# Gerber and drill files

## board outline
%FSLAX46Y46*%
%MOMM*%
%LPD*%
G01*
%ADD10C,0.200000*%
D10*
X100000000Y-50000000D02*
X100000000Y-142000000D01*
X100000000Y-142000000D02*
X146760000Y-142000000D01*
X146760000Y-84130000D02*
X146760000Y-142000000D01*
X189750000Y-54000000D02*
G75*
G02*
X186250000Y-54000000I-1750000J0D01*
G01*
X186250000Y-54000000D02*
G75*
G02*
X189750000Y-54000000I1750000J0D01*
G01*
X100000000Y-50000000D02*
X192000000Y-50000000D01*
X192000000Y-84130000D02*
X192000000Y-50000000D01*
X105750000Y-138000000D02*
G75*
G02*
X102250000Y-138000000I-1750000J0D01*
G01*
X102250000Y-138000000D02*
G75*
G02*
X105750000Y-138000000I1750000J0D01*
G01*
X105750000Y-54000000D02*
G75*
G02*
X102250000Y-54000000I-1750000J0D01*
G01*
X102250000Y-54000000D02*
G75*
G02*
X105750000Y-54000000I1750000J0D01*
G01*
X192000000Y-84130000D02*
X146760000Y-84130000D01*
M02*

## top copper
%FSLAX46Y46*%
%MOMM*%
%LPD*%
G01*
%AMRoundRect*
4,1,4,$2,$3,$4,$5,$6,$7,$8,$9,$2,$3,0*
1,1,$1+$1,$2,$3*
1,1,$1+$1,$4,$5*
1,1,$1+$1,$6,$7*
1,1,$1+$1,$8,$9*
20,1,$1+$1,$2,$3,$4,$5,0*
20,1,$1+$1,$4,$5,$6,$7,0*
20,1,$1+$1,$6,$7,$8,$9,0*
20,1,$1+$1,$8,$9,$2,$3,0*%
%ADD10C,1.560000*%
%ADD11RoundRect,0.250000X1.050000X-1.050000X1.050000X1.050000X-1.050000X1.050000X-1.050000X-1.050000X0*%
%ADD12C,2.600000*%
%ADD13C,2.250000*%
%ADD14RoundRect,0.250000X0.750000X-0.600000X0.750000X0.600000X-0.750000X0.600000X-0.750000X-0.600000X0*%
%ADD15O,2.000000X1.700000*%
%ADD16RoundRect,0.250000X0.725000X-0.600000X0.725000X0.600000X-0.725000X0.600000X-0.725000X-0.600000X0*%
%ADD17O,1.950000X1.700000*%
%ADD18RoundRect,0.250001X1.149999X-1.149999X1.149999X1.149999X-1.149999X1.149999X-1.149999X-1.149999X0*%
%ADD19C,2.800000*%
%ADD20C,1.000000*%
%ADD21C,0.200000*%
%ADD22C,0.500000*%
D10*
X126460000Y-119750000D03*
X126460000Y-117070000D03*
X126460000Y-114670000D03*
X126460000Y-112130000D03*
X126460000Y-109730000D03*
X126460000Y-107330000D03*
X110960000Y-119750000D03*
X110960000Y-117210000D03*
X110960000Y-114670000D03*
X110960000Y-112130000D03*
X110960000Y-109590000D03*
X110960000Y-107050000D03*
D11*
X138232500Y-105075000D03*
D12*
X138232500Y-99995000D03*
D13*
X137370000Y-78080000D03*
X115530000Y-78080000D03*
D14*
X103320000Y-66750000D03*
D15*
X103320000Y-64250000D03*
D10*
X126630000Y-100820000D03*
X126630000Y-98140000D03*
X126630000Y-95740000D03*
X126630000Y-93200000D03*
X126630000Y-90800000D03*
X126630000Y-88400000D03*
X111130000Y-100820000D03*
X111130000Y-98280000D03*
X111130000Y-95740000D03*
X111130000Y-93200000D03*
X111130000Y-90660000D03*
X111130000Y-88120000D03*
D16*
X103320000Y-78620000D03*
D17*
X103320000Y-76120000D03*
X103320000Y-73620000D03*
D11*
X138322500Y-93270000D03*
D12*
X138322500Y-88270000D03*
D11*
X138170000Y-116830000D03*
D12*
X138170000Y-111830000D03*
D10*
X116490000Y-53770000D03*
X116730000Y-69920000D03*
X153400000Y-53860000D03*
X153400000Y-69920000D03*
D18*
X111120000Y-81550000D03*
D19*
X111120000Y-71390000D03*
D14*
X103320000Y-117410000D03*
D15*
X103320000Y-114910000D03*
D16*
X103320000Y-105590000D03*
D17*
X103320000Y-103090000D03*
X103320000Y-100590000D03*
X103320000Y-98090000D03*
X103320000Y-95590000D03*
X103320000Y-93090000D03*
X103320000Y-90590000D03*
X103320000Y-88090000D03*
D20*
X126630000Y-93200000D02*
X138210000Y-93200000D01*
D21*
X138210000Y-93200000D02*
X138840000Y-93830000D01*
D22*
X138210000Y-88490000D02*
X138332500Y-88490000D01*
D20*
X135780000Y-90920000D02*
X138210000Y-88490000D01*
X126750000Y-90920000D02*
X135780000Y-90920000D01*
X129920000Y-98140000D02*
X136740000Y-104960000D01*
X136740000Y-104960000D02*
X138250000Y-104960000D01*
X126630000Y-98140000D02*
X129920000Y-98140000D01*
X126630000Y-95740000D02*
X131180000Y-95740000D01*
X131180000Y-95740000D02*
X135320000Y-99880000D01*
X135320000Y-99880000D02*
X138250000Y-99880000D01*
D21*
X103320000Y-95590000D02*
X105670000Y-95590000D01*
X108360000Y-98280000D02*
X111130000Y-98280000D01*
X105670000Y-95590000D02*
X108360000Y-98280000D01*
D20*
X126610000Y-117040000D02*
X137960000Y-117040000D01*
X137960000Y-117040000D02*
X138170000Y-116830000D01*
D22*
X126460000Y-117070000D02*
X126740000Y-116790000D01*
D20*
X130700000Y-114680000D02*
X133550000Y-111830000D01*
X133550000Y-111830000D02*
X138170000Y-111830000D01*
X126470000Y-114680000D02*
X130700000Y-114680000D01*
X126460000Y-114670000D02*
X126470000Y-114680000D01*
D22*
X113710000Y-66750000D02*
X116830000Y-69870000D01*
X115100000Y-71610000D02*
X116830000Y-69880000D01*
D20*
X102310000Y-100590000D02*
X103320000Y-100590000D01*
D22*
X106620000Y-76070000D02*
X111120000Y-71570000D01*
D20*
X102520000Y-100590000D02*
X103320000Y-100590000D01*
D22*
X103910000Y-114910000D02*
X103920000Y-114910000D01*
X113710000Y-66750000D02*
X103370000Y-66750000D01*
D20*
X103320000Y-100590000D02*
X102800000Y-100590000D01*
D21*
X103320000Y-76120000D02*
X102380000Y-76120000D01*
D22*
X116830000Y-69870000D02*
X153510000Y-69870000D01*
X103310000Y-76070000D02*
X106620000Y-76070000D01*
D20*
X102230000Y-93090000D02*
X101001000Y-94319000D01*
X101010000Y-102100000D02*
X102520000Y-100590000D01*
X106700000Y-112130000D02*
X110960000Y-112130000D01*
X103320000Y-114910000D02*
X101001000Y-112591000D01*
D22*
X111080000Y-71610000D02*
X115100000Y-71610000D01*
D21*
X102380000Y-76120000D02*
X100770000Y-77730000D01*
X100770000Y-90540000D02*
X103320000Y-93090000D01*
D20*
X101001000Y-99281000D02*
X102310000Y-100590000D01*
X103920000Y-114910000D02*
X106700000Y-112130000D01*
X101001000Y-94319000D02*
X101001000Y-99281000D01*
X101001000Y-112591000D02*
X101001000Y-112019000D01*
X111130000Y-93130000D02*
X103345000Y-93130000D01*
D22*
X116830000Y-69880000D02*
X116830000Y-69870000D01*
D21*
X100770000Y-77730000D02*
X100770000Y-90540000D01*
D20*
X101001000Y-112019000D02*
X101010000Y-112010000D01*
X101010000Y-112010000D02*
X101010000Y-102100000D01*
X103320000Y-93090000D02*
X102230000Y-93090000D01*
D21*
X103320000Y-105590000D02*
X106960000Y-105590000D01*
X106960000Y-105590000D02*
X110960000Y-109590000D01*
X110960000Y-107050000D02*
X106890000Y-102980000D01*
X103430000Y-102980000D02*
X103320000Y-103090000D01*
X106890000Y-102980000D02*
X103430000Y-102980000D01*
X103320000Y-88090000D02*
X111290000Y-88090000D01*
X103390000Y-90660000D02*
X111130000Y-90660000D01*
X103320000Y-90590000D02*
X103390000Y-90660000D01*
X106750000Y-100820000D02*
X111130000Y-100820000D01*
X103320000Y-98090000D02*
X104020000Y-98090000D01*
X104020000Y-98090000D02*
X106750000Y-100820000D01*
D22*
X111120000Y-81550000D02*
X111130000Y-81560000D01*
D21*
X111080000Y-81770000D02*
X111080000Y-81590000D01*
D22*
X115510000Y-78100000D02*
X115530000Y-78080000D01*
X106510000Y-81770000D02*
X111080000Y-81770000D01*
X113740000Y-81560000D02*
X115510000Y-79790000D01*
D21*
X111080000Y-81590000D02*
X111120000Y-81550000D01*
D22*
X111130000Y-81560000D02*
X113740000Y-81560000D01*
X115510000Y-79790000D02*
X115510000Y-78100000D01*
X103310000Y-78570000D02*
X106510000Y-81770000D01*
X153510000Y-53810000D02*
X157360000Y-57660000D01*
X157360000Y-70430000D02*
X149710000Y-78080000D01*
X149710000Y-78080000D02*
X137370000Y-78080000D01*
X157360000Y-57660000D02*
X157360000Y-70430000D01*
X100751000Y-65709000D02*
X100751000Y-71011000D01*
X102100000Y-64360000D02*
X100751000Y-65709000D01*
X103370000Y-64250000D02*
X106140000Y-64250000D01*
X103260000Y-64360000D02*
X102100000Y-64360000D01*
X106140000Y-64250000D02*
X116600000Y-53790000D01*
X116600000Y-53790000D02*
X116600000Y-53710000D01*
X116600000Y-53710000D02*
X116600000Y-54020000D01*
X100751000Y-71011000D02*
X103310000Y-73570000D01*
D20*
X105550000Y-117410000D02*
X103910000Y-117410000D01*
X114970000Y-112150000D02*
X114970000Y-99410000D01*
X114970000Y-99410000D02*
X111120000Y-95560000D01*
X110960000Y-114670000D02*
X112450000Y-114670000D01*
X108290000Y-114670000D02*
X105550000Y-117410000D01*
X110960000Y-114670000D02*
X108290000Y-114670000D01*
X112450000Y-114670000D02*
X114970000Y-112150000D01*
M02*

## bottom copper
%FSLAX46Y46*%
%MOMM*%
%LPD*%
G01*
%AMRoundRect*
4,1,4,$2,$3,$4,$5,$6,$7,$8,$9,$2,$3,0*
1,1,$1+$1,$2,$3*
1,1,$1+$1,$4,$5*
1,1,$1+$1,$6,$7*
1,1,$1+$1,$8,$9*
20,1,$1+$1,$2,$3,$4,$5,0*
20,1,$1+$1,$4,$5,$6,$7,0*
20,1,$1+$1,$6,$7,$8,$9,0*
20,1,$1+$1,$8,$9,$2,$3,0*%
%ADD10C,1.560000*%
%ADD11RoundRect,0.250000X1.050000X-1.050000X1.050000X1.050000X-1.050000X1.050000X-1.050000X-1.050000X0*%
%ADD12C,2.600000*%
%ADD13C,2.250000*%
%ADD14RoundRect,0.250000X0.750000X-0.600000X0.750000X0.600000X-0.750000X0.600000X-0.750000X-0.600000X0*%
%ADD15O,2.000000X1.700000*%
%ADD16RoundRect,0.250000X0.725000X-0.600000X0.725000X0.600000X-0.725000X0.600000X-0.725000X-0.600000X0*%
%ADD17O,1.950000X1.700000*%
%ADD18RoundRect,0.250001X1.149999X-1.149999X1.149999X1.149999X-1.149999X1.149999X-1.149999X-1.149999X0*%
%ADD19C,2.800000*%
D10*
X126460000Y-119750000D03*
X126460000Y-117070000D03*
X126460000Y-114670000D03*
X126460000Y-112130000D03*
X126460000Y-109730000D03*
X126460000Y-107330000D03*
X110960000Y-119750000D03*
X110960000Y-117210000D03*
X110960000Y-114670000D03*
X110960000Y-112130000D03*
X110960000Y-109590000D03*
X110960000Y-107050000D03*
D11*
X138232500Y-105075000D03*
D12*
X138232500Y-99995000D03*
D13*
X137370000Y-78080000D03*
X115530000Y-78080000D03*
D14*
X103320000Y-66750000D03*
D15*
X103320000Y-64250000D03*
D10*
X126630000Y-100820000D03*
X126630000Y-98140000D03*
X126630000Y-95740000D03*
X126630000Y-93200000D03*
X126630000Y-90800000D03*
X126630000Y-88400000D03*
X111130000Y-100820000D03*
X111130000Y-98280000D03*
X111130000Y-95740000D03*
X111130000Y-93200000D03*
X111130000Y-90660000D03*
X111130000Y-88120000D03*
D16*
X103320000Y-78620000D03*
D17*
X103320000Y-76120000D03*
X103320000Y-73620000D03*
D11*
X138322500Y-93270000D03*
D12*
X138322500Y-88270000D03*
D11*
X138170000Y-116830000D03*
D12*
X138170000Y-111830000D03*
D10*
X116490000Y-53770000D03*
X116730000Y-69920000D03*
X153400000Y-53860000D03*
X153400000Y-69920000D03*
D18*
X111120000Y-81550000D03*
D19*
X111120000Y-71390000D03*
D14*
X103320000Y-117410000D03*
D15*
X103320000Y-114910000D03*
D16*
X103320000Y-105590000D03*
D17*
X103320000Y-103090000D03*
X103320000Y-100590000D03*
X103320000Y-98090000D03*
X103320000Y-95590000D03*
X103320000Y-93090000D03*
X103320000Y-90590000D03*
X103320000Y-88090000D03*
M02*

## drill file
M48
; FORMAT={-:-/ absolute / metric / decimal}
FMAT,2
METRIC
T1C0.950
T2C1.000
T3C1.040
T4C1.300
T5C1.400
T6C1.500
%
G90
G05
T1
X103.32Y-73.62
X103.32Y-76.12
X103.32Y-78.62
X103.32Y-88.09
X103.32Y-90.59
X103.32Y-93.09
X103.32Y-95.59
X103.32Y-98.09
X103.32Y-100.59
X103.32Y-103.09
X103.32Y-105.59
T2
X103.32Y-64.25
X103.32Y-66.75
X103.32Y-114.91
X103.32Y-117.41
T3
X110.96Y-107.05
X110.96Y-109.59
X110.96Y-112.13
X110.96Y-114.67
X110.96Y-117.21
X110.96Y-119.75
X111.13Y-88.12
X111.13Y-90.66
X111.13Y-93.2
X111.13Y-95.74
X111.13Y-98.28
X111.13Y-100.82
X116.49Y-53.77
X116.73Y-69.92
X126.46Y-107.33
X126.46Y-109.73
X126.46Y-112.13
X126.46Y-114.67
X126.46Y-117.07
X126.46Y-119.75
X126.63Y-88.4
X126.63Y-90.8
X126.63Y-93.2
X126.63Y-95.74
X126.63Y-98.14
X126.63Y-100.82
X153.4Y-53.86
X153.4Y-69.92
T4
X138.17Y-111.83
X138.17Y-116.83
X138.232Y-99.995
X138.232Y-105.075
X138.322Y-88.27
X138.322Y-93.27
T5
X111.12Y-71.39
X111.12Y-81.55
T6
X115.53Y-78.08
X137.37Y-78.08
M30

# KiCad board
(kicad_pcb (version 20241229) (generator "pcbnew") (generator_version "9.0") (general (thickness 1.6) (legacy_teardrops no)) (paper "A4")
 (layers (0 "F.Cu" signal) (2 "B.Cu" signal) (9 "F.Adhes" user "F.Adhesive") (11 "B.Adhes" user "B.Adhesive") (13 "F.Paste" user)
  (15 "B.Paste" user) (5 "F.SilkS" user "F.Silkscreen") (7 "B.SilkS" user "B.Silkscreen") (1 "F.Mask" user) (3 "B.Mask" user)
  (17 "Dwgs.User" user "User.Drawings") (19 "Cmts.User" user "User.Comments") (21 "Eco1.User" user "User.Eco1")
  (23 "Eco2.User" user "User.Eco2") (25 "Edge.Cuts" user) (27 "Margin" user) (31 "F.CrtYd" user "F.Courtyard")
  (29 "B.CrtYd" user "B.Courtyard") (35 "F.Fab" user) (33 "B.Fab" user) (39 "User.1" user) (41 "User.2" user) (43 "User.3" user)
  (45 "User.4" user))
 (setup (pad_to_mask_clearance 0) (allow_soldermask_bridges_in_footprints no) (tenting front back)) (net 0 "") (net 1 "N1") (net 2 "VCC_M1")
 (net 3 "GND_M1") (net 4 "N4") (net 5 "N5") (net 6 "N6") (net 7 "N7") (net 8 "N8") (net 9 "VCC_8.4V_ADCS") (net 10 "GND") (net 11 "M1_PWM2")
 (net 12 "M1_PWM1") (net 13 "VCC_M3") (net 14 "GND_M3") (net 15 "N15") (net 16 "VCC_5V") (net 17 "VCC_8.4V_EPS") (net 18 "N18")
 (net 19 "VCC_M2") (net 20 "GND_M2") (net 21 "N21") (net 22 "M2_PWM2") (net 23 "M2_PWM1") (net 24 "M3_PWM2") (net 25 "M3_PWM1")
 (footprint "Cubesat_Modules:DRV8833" (layer "F.Cu") (at 118.71 113.4 180)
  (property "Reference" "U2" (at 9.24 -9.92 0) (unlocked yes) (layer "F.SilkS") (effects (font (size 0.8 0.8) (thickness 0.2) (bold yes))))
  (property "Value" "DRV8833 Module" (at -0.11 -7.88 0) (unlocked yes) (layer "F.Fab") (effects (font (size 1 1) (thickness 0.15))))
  (pad "1" thru_hole circle (at -7.75 -6.35 180) (size 1.56 1.56) (drill 1.04) (layers "*.Cu" "*.Mask") (remove_unused_layers no)
   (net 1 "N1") (solder_mask_margin 0.102))
  (pad "2" thru_hole circle (at -7.75 -3.67 180) (size 1.56 1.56) (drill 1.04) (layers "*.Cu" "*.Mask") (remove_unused_layers no)
   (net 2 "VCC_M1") (solder_mask_margin 0.102))
  (pad "3" thru_hole circle (at -7.75 -1.27 180) (size 1.56 1.56) (drill 1.04) (layers "*.Cu" "*.Mask") (remove_unused_layers no)
   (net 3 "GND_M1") (solder_mask_margin 0.102))
  (pad "4" thru_hole circle (at -7.75 1.27 180) (size 1.56 1.56) (drill 1.04) (layers "*.Cu" "*.Mask") (remove_unused_layers no)
   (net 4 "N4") (solder_mask_margin 0.102))
  (pad "5" thru_hole circle (at -7.75 3.67 180) (size 1.56 1.56) (drill 1.04) (layers "*.Cu" "*.Mask") (remove_unused_layers no)
   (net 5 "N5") (solder_mask_margin 0.102))
  (pad "6" thru_hole circle (at -7.75 6.07 180) (size 1.56 1.56) (drill 1.04) (layers "*.Cu" "*.Mask" "Eco2.User") (remove_unused_layers no)
   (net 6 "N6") (solder_mask_margin 0.102))
  (pad "7" thru_hole circle (at 7.75 -6.35 180) (size 1.56 1.56) (drill 1.04) (layers "*.Cu" "*.Mask") (remove_unused_layers no)
   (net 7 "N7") (solder_mask_margin 0.102))
  (pad "8" thru_hole circle (at 7.75 -3.81 180) (size 1.56 1.56) (drill 1.04) (layers "*.Cu" "*.Mask") (remove_unused_layers no)
   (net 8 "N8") (solder_mask_margin 0.102))
  (pad "9" thru_hole circle (at 7.75 -1.27 180) (size 1.56 1.56) (drill 1.04) (layers "*.Cu" "*.Mask") (remove_unused_layers no)
   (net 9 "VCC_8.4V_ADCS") (solder_mask_margin 0.102))
  (pad "10" thru_hole circle (at 7.75 1.27 180) (size 1.56 1.56) (drill 1.04) (layers "*.Cu" "*.Mask") (remove_unused_layers no)
   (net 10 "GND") (solder_mask_margin 0.102))
  (pad "11" thru_hole circle (at 7.75 3.81 180) (size 1.56 1.56) (drill 1.04) (layers "*.Cu" "*.Mask") (remove_unused_layers no)
   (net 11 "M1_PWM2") (solder_mask_margin 0.102))
  (pad "12" thru_hole circle (at 7.75 6.35 180) (size 1.56 1.56) (drill 1.04) (layers "*.Cu" "*.Mask") (remove_unused_layers no)
   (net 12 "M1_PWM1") (solder_mask_margin 0.102)))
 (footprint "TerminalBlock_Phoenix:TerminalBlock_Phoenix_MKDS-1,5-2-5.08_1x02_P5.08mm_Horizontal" (layer "F.Cu") (at 138.2325 105.075 90)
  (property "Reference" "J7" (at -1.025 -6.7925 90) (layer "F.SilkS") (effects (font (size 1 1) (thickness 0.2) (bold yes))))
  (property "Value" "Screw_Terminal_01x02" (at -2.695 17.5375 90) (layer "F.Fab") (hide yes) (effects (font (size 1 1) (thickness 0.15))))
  (pad "1" thru_hole roundrect (at 0 0 90) (size 2.6 2.6) (drill 1.3) (layers "*.Cu" "*.Mask") (remove_unused_layers no)
   (roundrect_rratio 0.096154) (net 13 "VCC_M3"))
  (pad "2" thru_hole circle (at 5.08 0 90) (size 2.6 2.6) (drill 1.3) (layers "*.Cu" "*.Mask") (remove_unused_layers no) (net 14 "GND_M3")))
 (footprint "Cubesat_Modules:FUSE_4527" (layer "F.Cu") (at 126.45 78.08 180)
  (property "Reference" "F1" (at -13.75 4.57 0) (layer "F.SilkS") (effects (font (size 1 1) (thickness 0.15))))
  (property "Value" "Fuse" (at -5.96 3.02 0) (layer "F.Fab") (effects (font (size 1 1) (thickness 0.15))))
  (pad "1" thru_hole circle (at -10.92 0 180) (size 2.25 2.25) (drill 1.5) (layers "*.Cu" "*.Mask") (remove_unused_layers no) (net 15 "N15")
   (solder_mask_margin 0.102))
  (pad "2" thru_hole circle (at 10.92 0 180) (size 2.25 2.25) (drill 1.5) (layers "*.Cu" "*.Mask") (remove_unused_layers no)
   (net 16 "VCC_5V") (solder_mask_margin 0.102)))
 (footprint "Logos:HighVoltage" (layer "F.Cu") (at 142.62 80.51)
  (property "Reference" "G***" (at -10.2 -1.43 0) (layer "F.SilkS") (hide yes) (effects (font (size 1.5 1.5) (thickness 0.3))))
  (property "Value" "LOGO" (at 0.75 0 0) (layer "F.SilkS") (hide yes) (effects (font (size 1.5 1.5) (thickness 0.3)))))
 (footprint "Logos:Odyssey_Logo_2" (layer "F.Cu") (at 132.96 138.74)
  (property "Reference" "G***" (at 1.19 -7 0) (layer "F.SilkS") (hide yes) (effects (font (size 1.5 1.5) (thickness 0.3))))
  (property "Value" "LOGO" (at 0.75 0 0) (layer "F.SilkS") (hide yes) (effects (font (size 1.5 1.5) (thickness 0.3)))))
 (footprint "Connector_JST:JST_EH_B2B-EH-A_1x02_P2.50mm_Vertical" (layer "F.Cu") (at 103.32 66.75 90)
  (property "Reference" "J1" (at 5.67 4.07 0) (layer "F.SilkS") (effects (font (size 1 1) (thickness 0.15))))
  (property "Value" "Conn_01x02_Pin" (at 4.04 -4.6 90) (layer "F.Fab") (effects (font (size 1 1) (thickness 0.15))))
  (pad "1" thru_hole roundrect (at 0 0 90) (size 1.7 2) (drill 1) (layers "*.Cu" "*.Mask") (remove_unused_layers no)
   (roundrect_rratio 0.147059) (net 10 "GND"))
  (pad "2" thru_hole oval (at 2.5 0 90) (size 1.7 2) (drill 1) (layers "*.Cu" "*.Mask") (remove_unused_layers no) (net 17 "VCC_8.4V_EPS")))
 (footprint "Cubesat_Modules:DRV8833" (layer "F.Cu") (at 118.88 94.47 180)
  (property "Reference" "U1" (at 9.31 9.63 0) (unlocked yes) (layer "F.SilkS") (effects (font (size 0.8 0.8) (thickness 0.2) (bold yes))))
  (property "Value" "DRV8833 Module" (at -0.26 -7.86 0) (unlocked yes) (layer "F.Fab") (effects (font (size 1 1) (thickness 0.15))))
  (pad "1" thru_hole circle (at -7.75 -6.35 180) (size 1.56 1.56) (drill 1.04) (layers "*.Cu" "*.Mask") (remove_unused_layers no)
   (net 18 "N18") (solder_mask_margin 0.102))
  (pad "2" thru_hole circle (at -7.75 -3.67 180) (size 1.56 1.56) (drill 1.04) (layers "*.Cu" "*.Mask") (remove_unused_layers no)
   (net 13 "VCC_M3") (solder_mask_margin 0.102))
  (pad "3" thru_hole circle (at -7.75 -1.27 180) (size 1.56 1.56) (drill 1.04) (layers "*.Cu" "*.Mask") (remove_unused_layers no)
   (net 14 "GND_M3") (solder_mask_margin 0.102))
  (pad "4" thru_hole circle (at -7.75 1.27 180) (size 1.56 1.56) (drill 1.04) (layers "*.Cu" "*.Mask") (remove_unused_layers no)
   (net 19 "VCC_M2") (solder_mask_margin 0.102))
  (pad "5" thru_hole circle (at -7.75 3.67 180) (size 1.56 1.56) (drill 1.04) (layers "*.Cu" "*.Mask") (remove_unused_layers no)
   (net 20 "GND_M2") (solder_mask_margin 0.102))
  (pad "6" thru_hole circle (at -7.75 6.07 180) (size 1.56 1.56) (drill 1.04) (layers "*.Cu" "*.Mask" "Eco2.User") (remove_unused_layers no)
   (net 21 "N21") (solder_mask_margin 0.102))
  (pad "7" thru_hole circle (at 7.75 -6.35 180) (size 1.56 1.56) (drill 1.04) (layers "*.Cu" "*.Mask") (remove_unused_layers no)
   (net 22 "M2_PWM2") (solder_mask_margin 0.102))
  (pad "8" thru_hole circle (at 7.75 -3.81 180) (size 1.56 1.56) (drill 1.04) (layers "*.Cu" "*.Mask") (remove_unused_layers no)
   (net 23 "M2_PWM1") (solder_mask_margin 0.102))
  (pad "9" thru_hole circle (at 7.75 -1.27 180) (size 1.56 1.56) (drill 1.04) (layers "*.Cu" "*.Mask") (remove_unused_layers no)
   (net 9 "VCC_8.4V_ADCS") (solder_mask_margin 0.102))
  (pad "10" thru_hole circle (at 7.75 1.27 180) (size 1.56 1.56) (drill 1.04) (layers "*.Cu" "*.Mask") (remove_unused_layers no)
   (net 10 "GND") (solder_mask_margin 0.102))
  (pad "11" thru_hole circle (at 7.75 3.81 180) (size 1.56 1.56) (drill 1.04) (layers "*.Cu" "*.Mask") (remove_unused_layers no)
   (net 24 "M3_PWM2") (solder_mask_margin 0.102))
  (pad "12" thru_hole circle (at 7.75 6.35 180) (size 1.56 1.56) (drill 1.04) (layers "*.Cu" "*.Mask") (remove_unused_layers no)
   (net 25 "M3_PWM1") (solder_mask_margin 0.102)))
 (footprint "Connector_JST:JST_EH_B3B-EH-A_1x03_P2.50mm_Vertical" (layer "F.Cu") (at 103.32 78.62 90)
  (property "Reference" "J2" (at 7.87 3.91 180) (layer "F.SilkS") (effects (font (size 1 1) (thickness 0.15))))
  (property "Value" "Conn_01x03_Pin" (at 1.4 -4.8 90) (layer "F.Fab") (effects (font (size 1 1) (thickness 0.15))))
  (pad "1" thru_hole roundrect (at 0 0 90) (size 1.7 1.95) (drill 0.95) (layers "*.Cu" "*.Mask") (remove_unused_layers no)
   (roundrect_rratio 0.147059) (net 16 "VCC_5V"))
  (pad "2" thru_hole oval (at 2.5 0 90) (size 1.7 1.95) (drill 0.95) (layers "*.Cu" "*.Mask") (remove_unused_layers no) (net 10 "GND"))
  (pad "3" thru_hole oval (at 5 0 90) (size 1.7 1.95) (drill 0.95) (layers "*.Cu" "*.Mask") (remove_unused_layers no)
   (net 17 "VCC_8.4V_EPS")))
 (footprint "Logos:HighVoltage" (layer "F.Cu") (at 163.1 54)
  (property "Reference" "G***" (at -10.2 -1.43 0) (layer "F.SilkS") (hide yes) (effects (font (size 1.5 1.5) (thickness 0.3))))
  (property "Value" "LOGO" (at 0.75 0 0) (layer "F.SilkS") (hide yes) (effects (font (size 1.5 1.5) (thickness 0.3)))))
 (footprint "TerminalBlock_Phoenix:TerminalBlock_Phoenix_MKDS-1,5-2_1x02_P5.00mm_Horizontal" (layer "F.Cu") (at 138.3225 93.27 90)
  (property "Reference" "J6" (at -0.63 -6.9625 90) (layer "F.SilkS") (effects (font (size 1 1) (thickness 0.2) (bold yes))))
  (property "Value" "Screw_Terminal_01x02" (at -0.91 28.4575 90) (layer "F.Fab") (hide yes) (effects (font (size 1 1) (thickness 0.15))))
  (pad "1" thru_hole roundrect (at 0 0 90) (size 2.6 2.6) (drill 1.3) (layers "*.Cu" "*.Mask") (remove_unused_layers no)
   (roundrect_rratio 0.096154) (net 19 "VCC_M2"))
  (pad "2" thru_hole circle (at 5 0 90) (size 2.6 2.6) (drill 1.3) (layers "*.Cu" "*.Mask") (remove_unused_layers no) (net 20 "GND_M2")))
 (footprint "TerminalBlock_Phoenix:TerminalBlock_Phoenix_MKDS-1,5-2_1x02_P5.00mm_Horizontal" (layer "F.Cu") (at 138.17 116.83 90)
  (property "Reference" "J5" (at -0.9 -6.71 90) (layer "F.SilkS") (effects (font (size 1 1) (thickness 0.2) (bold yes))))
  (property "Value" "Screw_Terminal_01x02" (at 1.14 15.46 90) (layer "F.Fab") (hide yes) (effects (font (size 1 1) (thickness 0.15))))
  (pad "1" thru_hole roundrect (at 0 0 90) (size 2.6 2.6) (drill 1.3) (layers "*.Cu" "*.Mask") (remove_unused_layers no)
   (roundrect_rratio 0.096154) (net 2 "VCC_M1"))
  (pad "2" thru_hole circle (at 5 0 90) (size 2.6 2.6) (drill 1.3) (layers "*.Cu" "*.Mask") (remove_unused_layers no) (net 3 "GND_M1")))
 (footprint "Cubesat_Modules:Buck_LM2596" (layer "F.Cu") (at 135.07 61.89 -90)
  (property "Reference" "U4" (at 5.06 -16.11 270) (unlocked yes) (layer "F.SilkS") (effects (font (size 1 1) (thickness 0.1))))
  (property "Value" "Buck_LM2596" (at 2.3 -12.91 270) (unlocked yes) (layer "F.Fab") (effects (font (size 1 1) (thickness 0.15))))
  (pad "1" thru_hole circle (at -8.12 18.58) (size 1.56 1.56) (drill 1.04) (layers "*.Cu" "*.Mask") (remove_unused_layers no)
   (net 17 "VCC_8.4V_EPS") (solder_mask_margin 0.102))
  (pad "2" thru_hole circle (at 8.03 18.34) (size 1.56 1.56) (drill 1.04) (layers "*.Cu" "*.Mask") (remove_unused_layers no) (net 10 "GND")
   (solder_mask_margin 0.102))
  (pad "3" thru_hole circle (at -8.03 -18.33) (size 1.56 1.56) (drill 1.04) (layers "*.Cu" "*.Mask") (remove_unused_layers no)
   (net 15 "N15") (solder_mask_margin 0.102))
  (pad "4" thru_hole circle (at 8.03 -18.33) (size 1.56 1.56) (drill 1.04) (layers "*.Cu" "*.Mask") (remove_unused_layers no) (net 10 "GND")
   (solder_mask_margin 0.102)))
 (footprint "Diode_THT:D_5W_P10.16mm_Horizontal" (layer "F.Cu") (at 111.12 81.55 90)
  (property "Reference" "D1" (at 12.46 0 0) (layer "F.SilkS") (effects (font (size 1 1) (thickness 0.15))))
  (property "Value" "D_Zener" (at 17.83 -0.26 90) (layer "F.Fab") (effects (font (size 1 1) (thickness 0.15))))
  (pad "1" thru_hole roundrect (at 0 0 90) (size 2.8 2.8) (drill 1.4) (layers "*.Cu" "*.Mask") (remove_unused_layers no)
   (roundrect_rratio 0.089286) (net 16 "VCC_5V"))
  (pad "2" thru_hole circle (at 10.16 0 90) (size 2.8 2.8) (drill 1.4) (layers "*.Cu" "*.Mask") (remove_unused_layers no) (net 10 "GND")))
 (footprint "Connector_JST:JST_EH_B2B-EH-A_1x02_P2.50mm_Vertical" (layer "F.Cu") (at 103.32 117.41 90)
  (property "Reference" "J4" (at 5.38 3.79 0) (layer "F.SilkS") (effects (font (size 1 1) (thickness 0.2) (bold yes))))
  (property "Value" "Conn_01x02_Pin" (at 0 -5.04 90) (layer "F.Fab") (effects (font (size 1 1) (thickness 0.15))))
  (pad "1" thru_hole roundrect (at 0 0 90) (size 1.7 2) (drill 1) (layers "*.Cu" "*.Mask") (remove_unused_layers no)
   (roundrect_rratio 0.147059) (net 9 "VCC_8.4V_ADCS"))
  (pad "2" thru_hole oval (at 2.5 0 90) (size 1.7 2) (drill 1) (layers "*.Cu" "*.Mask") (remove_unused_layers no) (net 10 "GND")))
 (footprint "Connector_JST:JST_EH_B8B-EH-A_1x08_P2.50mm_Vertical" (layer "F.Cu") (at 103.32 105.59 90)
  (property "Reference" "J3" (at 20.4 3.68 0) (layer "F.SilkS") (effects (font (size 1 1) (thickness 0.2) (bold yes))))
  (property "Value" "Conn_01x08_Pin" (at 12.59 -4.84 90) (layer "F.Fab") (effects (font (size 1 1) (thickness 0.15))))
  (pad "1" thru_hole roundrect (at 0 0 90) (size 1.7 1.95) (drill 0.95) (layers "*.Cu" "*.Mask") (remove_unused_layers no)
   (roundrect_rratio 0.147059) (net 11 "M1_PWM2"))
  (pad "2" thru_hole oval (at 2.5 0 90) (size 1.7 1.95) (drill 0.95) (layers "*.Cu" "*.Mask") (remove_unused_layers no) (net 12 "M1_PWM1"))
  (pad "3" thru_hole oval (at 5 0 90) (size 1.7 1.95) (drill 0.95) (layers "*.Cu" "*.Mask") (remove_unused_layers no) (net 10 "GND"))
  (pad "4" thru_hole oval (at 7.5 0 90) (size 1.7 1.95) (drill 0.95) (layers "*.Cu" "*.Mask") (remove_unused_layers no) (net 22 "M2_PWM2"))
  (pad "5" thru_hole oval (at 10 0 90) (size 1.7 1.95) (drill 0.95) (layers "*.Cu" "*.Mask") (remove_unused_layers no) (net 23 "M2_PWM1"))
  (pad "6" thru_hole oval (at 12.5 0 90) (size 1.7 1.95) (drill 0.95) (layers "*.Cu" "*.Mask") (remove_unused_layers no) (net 10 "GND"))
  (pad "7" thru_hole oval (at 15 0 90) (size 1.7 1.95) (drill 0.95) (layers "*.Cu" "*.Mask") (remove_unused_layers no) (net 24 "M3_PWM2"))
  (pad "8" thru_hole oval (at 17.5 0 90) (size 1.7 1.95) (drill 0.95) (layers "*.Cu" "*.Mask") (remove_unused_layers no) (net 25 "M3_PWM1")))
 (gr_line (start 100 50) (end 100 142) (stroke (width 0.2) (type solid)) (layer "Edge.Cuts"))
 (gr_line (start 100 142) (end 146.76 142) (stroke (width 0.2) (type solid)) (layer "Edge.Cuts"))
 (gr_line (start 146.76 84.13) (end 146.76 142) (stroke (width 0.2) (type solid)) (layer "Edge.Cuts"))
 (gr_circle (center 188 54) (end 189.75 54) (stroke (width 0.2) (type solid)) (fill no) (layer "Edge.Cuts"))
 (gr_line (start 100 50) (end 192 50) (stroke (width 0.2) (type solid)) (layer "Edge.Cuts"))
 (gr_line (start 192 84.13) (end 192 50) (stroke (width 0.2) (type solid)) (layer "Edge.Cuts"))
 (gr_circle (center 104 138) (end 105.75 138) (stroke (width 0.2) (type solid)) (fill no) (layer "Edge.Cuts"))
 (gr_circle (center 104 54) (end 105.75 54) (stroke (width 0.2) (type solid)) (fill no) (layer "Edge.Cuts"))
 (gr_line (start 192 84.13) (end 146.76 84.13) (stroke (width 0.2) (type solid)) (layer "Edge.Cuts"))
 (segment (start 126.63 93.2) (end 138.21 93.2) (width 1) (layer "F.Cu") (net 19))
 (segment (start 138.21 93.2) (end 138.84 93.83) (width 0.2) (layer "F.Cu") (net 19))
 (segment (start 138.21 88.49) (end 138.3325 88.49) (width 0.5) (layer "F.Cu") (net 20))
 (segment (start 135.78 90.92) (end 138.21 88.49) (width 1) (layer "F.Cu") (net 20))
 (segment (start 126.75 90.92) (end 135.78 90.92) (width 1) (layer "F.Cu") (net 20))
 (segment (start 129.92 98.14) (end 136.74 104.96) (width 1) (layer "F.Cu") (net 13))
 (segment (start 136.74 104.96) (end 138.25 104.96) (width 1) (layer "F.Cu") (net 13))
 (segment (start 126.63 98.14) (end 129.92 98.14) (width 1) (layer "F.Cu") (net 13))
 (segment (start 126.63 95.74) (end 131.18 95.74) (width 1) (layer "F.Cu") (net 14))
 (segment (start 131.18 95.74) (end 135.32 99.88) (width 1) (layer "F.Cu") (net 14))
 (segment (start 135.32 99.88) (end 138.25 99.88) (width 1) (layer "F.Cu") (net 14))
 (segment (start 103.32 95.59) (end 105.67 95.59) (width 0.2) (layer "F.Cu") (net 23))
 (segment (start 108.36 98.28) (end 111.13 98.28) (width 0.2) (layer "F.Cu") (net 23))
 (segment (start 105.67 95.59) (end 108.36 98.28) (width 0.2) (layer "F.Cu") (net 23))
 (segment (start 126.61 117.04) (end 137.96 117.04) (width 1) (layer "F.Cu") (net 2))
 (segment (start 137.96 117.04) (end 138.17 116.83) (width 1) (layer "F.Cu") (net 2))
 (segment (start 126.46 117.07) (end 126.74 116.79) (width 0.5) (layer "F.Cu") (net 2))
 (segment (start 130.7 114.68) (end 133.55 111.83) (width 1) (layer "F.Cu") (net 3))
 (segment (start 133.55 111.83) (end 138.17 111.83) (width 1) (layer "F.Cu") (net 3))
 (segment (start 126.47 114.68) (end 130.7 114.68) (width 1) (layer "F.Cu") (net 3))
 (segment (start 126.46 114.67) (end 126.47 114.68) (width 1) (layer "F.Cu") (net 3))
 (segment (start 113.71 66.75) (end 116.83 69.87) (width 0.5) (layer "F.Cu") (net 10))
 (segment (start 115.1 71.61) (end 116.83 69.88) (width 0.5) (layer "F.Cu") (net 10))
 (segment (start 102.31 100.59) (end 103.32 100.59) (width 1) (layer "F.Cu") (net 10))
 (segment (start 106.62 76.07) (end 111.12 71.57) (width 0.5) (layer "F.Cu") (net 10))
 (segment (start 102.52 100.59) (end 103.32 100.59) (width 1) (layer "F.Cu") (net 10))
 (segment (start 103.91 114.91) (end 103.92 114.91) (width 0.5) (layer "F.Cu") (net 10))
 (segment (start 113.71 66.75) (end 103.37 66.75) (width 0.5) (layer "F.Cu") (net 10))
 (segment (start 103.32 100.59) (end 102.8 100.59) (width 1) (layer "F.Cu") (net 10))
 (segment (start 103.32 76.12) (end 102.38 76.12) (width 0.2) (layer "F.Cu") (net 10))
 (segment (start 116.83 69.87) (end 153.51 69.87) (width 0.5) (layer "F.Cu") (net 10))
 (segment (start 103.31 76.07) (end 106.62 76.07) (width 0.5) (layer "F.Cu") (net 10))
 (segment (start 102.23 93.09) (end 101.001 94.319) (width 1) (layer "F.Cu") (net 10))
 (segment (start 101.01 102.1) (end 102.52 100.59) (width 1) (layer "F.Cu") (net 10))
 (segment (start 106.7 112.13) (end 110.96 112.13) (width 1) (layer "F.Cu") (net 10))
 (segment (start 103.32 114.91) (end 101.001 112.591) (width 1) (layer "F.Cu") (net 10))
 (segment (start 111.08 71.61) (end 115.1 71.61) (width 0.5) (layer "F.Cu") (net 10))
 (segment (start 102.38 76.12) (end 100.77 77.73) (width 0.2) (layer "F.Cu") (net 10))
 (segment (start 100.77 90.54) (end 103.32 93.09) (width 0.2) (layer "F.Cu") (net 10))
 (segment (start 101.001 99.281) (end 102.31 100.59) (width 1) (layer "F.Cu") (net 10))
 (segment (start 103.92 114.91) (end 106.7 112.13) (width 1) (layer "F.Cu") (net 10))
 (segment (start 101.001 94.319) (end 101.001 99.281) (width 1) (layer "F.Cu") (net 10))
 (segment (start 101.001 112.591) (end 101.001 112.019) (width 1) (layer "F.Cu") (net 10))
 (segment (start 111.13 93.13) (end 103.345 93.13) (width 1) (layer "F.Cu") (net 10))
 (segment (start 116.83 69.88) (end 116.83 69.87) (width 0.5) (layer "F.Cu") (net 10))
 (segment (start 100.77 77.73) (end 100.77 90.54) (width 0.2) (layer "F.Cu") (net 10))
 (segment (start 101.001 112.019) (end 101.01 112.01) (width 1) (layer "F.Cu") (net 10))
 (segment (start 101.01 112.01) (end 101.01 102.1) (width 1) (layer "F.Cu") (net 10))
 (segment (start 103.32 93.09) (end 102.23 93.09) (width 1) (layer "F.Cu") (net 10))
 (segment (start 103.32 105.59) (end 106.96 105.59) (width 0.2) (layer "F.Cu") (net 11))
 (segment (start 106.96 105.59) (end 110.96 109.59) (width 0.2) (layer "F.Cu") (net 11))
 (segment (start 110.96 107.05) (end 106.89 102.98) (width 0.2) (layer "F.Cu") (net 12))
 (segment (start 103.43 102.98) (end 103.32 103.09) (width 0.2) (layer "F.Cu") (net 12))
 (segment (start 106.89 102.98) (end 103.43 102.98) (width 0.2) (layer "F.Cu") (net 12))
 (segment (start 103.32 88.09) (end 111.29 88.09) (width 0.2) (layer "F.Cu") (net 25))
 (segment (start 103.39 90.66) (end 111.13 90.66) (width 0.2) (layer "F.Cu") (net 24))
 (segment (start 103.32 90.59) (end 103.39 90.66) (width 0.2) (layer "F.Cu") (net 24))
 (segment (start 106.75 100.82) (end 111.13 100.82) (width 0.2) (layer "F.Cu") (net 22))
 (segment (start 103.32 98.09) (end 104.02 98.09) (width 0.2) (layer "F.Cu") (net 22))
 (segment (start 104.02 98.09) (end 106.75 100.82) (width 0.2) (layer "F.Cu") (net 22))
 (segment (start 111.12 81.55) (end 111.13 81.56) (width 0.5) (layer "F.Cu") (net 16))
 (segment (start 111.08 81.77) (end 111.08 81.59) (width 0.2) (layer "F.Cu") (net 16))
 (segment (start 115.51 78.1) (end 115.53 78.08) (width 0.5) (layer "F.Cu") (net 16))
 (segment (start 106.51 81.77) (end 111.08 81.77) (width 0.5) (layer "F.Cu") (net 16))
 (segment (start 113.74 81.56) (end 115.51 79.79) (width 0.5) (layer "F.Cu") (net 16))
 (segment (start 111.08 81.59) (end 111.12 81.55) (width 0.2) (layer "F.Cu") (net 16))
 (segment (start 111.13 81.56) (end 113.74 81.56) (width 0.5) (layer "F.Cu") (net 16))
 (segment (start 115.51 79.79) (end 115.51 78.1) (width 0.5) (layer "F.Cu") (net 16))
 (segment (start 103.31 78.57) (end 106.51 81.77) (width 0.5) (layer "F.Cu") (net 16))
 (segment (start 153.51 53.81) (end 157.36 57.66) (width 0.5) (layer "F.Cu") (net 15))
 (segment (start 157.36 70.43) (end 149.71 78.08) (width 0.5) (layer "F.Cu") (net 15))
 (segment (start 149.71 78.08) (end 137.37 78.08) (width 0.5) (layer "F.Cu") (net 15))
 (segment (start 157.36 57.66) (end 157.36 70.43) (width 0.5) (layer "F.Cu") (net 15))
 (segment (start 100.751 65.709) (end 100.751 71.011) (width 0.5) (layer "F.Cu") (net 17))
 (segment (start 102.1 64.36) (end 100.751 65.709) (width 0.5) (layer "F.Cu") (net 17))
 (segment (start 103.37 64.25) (end 106.14 64.25) (width 0.5) (layer "F.Cu") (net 17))
 (segment (start 103.26 64.36) (end 102.1 64.36) (width 0.5) (layer "F.Cu") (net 17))
 (segment (start 106.14 64.25) (end 116.6 53.79) (width 0.5) (layer "F.Cu") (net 17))
 (segment (start 116.6 53.79) (end 116.6 53.71) (width 0.5) (layer "F.Cu") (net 17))
 (segment (start 116.6 53.71) (end 116.6 54.02) (width 0.5) (layer "F.Cu") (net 17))
 (segment (start 100.751 71.011) (end 103.31 73.57) (width 0.5) (layer "F.Cu") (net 17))
 (segment (start 105.55 117.41) (end 103.91 117.41) (width 1) (layer "F.Cu") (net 9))
 (segment (start 114.97 112.15) (end 114.97 99.41) (width 1) (layer "F.Cu") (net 9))
 (segment (start 114.97 99.41) (end 111.12 95.56) (width 1) (layer "F.Cu") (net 9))
 (segment (start 110.96 114.67) (end 112.45 114.67) (width 1) (layer "F.Cu") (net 9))
 (segment (start 108.29 114.67) (end 105.55 117.41) (width 1) (layer "F.Cu") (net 9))
 (segment (start 110.96 114.67) (end 108.29 114.67) (width 1) (layer "F.Cu") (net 9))
 (segment (start 112.45 114.67) (end 114.97 112.15) (width 1) (layer "F.Cu") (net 9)))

